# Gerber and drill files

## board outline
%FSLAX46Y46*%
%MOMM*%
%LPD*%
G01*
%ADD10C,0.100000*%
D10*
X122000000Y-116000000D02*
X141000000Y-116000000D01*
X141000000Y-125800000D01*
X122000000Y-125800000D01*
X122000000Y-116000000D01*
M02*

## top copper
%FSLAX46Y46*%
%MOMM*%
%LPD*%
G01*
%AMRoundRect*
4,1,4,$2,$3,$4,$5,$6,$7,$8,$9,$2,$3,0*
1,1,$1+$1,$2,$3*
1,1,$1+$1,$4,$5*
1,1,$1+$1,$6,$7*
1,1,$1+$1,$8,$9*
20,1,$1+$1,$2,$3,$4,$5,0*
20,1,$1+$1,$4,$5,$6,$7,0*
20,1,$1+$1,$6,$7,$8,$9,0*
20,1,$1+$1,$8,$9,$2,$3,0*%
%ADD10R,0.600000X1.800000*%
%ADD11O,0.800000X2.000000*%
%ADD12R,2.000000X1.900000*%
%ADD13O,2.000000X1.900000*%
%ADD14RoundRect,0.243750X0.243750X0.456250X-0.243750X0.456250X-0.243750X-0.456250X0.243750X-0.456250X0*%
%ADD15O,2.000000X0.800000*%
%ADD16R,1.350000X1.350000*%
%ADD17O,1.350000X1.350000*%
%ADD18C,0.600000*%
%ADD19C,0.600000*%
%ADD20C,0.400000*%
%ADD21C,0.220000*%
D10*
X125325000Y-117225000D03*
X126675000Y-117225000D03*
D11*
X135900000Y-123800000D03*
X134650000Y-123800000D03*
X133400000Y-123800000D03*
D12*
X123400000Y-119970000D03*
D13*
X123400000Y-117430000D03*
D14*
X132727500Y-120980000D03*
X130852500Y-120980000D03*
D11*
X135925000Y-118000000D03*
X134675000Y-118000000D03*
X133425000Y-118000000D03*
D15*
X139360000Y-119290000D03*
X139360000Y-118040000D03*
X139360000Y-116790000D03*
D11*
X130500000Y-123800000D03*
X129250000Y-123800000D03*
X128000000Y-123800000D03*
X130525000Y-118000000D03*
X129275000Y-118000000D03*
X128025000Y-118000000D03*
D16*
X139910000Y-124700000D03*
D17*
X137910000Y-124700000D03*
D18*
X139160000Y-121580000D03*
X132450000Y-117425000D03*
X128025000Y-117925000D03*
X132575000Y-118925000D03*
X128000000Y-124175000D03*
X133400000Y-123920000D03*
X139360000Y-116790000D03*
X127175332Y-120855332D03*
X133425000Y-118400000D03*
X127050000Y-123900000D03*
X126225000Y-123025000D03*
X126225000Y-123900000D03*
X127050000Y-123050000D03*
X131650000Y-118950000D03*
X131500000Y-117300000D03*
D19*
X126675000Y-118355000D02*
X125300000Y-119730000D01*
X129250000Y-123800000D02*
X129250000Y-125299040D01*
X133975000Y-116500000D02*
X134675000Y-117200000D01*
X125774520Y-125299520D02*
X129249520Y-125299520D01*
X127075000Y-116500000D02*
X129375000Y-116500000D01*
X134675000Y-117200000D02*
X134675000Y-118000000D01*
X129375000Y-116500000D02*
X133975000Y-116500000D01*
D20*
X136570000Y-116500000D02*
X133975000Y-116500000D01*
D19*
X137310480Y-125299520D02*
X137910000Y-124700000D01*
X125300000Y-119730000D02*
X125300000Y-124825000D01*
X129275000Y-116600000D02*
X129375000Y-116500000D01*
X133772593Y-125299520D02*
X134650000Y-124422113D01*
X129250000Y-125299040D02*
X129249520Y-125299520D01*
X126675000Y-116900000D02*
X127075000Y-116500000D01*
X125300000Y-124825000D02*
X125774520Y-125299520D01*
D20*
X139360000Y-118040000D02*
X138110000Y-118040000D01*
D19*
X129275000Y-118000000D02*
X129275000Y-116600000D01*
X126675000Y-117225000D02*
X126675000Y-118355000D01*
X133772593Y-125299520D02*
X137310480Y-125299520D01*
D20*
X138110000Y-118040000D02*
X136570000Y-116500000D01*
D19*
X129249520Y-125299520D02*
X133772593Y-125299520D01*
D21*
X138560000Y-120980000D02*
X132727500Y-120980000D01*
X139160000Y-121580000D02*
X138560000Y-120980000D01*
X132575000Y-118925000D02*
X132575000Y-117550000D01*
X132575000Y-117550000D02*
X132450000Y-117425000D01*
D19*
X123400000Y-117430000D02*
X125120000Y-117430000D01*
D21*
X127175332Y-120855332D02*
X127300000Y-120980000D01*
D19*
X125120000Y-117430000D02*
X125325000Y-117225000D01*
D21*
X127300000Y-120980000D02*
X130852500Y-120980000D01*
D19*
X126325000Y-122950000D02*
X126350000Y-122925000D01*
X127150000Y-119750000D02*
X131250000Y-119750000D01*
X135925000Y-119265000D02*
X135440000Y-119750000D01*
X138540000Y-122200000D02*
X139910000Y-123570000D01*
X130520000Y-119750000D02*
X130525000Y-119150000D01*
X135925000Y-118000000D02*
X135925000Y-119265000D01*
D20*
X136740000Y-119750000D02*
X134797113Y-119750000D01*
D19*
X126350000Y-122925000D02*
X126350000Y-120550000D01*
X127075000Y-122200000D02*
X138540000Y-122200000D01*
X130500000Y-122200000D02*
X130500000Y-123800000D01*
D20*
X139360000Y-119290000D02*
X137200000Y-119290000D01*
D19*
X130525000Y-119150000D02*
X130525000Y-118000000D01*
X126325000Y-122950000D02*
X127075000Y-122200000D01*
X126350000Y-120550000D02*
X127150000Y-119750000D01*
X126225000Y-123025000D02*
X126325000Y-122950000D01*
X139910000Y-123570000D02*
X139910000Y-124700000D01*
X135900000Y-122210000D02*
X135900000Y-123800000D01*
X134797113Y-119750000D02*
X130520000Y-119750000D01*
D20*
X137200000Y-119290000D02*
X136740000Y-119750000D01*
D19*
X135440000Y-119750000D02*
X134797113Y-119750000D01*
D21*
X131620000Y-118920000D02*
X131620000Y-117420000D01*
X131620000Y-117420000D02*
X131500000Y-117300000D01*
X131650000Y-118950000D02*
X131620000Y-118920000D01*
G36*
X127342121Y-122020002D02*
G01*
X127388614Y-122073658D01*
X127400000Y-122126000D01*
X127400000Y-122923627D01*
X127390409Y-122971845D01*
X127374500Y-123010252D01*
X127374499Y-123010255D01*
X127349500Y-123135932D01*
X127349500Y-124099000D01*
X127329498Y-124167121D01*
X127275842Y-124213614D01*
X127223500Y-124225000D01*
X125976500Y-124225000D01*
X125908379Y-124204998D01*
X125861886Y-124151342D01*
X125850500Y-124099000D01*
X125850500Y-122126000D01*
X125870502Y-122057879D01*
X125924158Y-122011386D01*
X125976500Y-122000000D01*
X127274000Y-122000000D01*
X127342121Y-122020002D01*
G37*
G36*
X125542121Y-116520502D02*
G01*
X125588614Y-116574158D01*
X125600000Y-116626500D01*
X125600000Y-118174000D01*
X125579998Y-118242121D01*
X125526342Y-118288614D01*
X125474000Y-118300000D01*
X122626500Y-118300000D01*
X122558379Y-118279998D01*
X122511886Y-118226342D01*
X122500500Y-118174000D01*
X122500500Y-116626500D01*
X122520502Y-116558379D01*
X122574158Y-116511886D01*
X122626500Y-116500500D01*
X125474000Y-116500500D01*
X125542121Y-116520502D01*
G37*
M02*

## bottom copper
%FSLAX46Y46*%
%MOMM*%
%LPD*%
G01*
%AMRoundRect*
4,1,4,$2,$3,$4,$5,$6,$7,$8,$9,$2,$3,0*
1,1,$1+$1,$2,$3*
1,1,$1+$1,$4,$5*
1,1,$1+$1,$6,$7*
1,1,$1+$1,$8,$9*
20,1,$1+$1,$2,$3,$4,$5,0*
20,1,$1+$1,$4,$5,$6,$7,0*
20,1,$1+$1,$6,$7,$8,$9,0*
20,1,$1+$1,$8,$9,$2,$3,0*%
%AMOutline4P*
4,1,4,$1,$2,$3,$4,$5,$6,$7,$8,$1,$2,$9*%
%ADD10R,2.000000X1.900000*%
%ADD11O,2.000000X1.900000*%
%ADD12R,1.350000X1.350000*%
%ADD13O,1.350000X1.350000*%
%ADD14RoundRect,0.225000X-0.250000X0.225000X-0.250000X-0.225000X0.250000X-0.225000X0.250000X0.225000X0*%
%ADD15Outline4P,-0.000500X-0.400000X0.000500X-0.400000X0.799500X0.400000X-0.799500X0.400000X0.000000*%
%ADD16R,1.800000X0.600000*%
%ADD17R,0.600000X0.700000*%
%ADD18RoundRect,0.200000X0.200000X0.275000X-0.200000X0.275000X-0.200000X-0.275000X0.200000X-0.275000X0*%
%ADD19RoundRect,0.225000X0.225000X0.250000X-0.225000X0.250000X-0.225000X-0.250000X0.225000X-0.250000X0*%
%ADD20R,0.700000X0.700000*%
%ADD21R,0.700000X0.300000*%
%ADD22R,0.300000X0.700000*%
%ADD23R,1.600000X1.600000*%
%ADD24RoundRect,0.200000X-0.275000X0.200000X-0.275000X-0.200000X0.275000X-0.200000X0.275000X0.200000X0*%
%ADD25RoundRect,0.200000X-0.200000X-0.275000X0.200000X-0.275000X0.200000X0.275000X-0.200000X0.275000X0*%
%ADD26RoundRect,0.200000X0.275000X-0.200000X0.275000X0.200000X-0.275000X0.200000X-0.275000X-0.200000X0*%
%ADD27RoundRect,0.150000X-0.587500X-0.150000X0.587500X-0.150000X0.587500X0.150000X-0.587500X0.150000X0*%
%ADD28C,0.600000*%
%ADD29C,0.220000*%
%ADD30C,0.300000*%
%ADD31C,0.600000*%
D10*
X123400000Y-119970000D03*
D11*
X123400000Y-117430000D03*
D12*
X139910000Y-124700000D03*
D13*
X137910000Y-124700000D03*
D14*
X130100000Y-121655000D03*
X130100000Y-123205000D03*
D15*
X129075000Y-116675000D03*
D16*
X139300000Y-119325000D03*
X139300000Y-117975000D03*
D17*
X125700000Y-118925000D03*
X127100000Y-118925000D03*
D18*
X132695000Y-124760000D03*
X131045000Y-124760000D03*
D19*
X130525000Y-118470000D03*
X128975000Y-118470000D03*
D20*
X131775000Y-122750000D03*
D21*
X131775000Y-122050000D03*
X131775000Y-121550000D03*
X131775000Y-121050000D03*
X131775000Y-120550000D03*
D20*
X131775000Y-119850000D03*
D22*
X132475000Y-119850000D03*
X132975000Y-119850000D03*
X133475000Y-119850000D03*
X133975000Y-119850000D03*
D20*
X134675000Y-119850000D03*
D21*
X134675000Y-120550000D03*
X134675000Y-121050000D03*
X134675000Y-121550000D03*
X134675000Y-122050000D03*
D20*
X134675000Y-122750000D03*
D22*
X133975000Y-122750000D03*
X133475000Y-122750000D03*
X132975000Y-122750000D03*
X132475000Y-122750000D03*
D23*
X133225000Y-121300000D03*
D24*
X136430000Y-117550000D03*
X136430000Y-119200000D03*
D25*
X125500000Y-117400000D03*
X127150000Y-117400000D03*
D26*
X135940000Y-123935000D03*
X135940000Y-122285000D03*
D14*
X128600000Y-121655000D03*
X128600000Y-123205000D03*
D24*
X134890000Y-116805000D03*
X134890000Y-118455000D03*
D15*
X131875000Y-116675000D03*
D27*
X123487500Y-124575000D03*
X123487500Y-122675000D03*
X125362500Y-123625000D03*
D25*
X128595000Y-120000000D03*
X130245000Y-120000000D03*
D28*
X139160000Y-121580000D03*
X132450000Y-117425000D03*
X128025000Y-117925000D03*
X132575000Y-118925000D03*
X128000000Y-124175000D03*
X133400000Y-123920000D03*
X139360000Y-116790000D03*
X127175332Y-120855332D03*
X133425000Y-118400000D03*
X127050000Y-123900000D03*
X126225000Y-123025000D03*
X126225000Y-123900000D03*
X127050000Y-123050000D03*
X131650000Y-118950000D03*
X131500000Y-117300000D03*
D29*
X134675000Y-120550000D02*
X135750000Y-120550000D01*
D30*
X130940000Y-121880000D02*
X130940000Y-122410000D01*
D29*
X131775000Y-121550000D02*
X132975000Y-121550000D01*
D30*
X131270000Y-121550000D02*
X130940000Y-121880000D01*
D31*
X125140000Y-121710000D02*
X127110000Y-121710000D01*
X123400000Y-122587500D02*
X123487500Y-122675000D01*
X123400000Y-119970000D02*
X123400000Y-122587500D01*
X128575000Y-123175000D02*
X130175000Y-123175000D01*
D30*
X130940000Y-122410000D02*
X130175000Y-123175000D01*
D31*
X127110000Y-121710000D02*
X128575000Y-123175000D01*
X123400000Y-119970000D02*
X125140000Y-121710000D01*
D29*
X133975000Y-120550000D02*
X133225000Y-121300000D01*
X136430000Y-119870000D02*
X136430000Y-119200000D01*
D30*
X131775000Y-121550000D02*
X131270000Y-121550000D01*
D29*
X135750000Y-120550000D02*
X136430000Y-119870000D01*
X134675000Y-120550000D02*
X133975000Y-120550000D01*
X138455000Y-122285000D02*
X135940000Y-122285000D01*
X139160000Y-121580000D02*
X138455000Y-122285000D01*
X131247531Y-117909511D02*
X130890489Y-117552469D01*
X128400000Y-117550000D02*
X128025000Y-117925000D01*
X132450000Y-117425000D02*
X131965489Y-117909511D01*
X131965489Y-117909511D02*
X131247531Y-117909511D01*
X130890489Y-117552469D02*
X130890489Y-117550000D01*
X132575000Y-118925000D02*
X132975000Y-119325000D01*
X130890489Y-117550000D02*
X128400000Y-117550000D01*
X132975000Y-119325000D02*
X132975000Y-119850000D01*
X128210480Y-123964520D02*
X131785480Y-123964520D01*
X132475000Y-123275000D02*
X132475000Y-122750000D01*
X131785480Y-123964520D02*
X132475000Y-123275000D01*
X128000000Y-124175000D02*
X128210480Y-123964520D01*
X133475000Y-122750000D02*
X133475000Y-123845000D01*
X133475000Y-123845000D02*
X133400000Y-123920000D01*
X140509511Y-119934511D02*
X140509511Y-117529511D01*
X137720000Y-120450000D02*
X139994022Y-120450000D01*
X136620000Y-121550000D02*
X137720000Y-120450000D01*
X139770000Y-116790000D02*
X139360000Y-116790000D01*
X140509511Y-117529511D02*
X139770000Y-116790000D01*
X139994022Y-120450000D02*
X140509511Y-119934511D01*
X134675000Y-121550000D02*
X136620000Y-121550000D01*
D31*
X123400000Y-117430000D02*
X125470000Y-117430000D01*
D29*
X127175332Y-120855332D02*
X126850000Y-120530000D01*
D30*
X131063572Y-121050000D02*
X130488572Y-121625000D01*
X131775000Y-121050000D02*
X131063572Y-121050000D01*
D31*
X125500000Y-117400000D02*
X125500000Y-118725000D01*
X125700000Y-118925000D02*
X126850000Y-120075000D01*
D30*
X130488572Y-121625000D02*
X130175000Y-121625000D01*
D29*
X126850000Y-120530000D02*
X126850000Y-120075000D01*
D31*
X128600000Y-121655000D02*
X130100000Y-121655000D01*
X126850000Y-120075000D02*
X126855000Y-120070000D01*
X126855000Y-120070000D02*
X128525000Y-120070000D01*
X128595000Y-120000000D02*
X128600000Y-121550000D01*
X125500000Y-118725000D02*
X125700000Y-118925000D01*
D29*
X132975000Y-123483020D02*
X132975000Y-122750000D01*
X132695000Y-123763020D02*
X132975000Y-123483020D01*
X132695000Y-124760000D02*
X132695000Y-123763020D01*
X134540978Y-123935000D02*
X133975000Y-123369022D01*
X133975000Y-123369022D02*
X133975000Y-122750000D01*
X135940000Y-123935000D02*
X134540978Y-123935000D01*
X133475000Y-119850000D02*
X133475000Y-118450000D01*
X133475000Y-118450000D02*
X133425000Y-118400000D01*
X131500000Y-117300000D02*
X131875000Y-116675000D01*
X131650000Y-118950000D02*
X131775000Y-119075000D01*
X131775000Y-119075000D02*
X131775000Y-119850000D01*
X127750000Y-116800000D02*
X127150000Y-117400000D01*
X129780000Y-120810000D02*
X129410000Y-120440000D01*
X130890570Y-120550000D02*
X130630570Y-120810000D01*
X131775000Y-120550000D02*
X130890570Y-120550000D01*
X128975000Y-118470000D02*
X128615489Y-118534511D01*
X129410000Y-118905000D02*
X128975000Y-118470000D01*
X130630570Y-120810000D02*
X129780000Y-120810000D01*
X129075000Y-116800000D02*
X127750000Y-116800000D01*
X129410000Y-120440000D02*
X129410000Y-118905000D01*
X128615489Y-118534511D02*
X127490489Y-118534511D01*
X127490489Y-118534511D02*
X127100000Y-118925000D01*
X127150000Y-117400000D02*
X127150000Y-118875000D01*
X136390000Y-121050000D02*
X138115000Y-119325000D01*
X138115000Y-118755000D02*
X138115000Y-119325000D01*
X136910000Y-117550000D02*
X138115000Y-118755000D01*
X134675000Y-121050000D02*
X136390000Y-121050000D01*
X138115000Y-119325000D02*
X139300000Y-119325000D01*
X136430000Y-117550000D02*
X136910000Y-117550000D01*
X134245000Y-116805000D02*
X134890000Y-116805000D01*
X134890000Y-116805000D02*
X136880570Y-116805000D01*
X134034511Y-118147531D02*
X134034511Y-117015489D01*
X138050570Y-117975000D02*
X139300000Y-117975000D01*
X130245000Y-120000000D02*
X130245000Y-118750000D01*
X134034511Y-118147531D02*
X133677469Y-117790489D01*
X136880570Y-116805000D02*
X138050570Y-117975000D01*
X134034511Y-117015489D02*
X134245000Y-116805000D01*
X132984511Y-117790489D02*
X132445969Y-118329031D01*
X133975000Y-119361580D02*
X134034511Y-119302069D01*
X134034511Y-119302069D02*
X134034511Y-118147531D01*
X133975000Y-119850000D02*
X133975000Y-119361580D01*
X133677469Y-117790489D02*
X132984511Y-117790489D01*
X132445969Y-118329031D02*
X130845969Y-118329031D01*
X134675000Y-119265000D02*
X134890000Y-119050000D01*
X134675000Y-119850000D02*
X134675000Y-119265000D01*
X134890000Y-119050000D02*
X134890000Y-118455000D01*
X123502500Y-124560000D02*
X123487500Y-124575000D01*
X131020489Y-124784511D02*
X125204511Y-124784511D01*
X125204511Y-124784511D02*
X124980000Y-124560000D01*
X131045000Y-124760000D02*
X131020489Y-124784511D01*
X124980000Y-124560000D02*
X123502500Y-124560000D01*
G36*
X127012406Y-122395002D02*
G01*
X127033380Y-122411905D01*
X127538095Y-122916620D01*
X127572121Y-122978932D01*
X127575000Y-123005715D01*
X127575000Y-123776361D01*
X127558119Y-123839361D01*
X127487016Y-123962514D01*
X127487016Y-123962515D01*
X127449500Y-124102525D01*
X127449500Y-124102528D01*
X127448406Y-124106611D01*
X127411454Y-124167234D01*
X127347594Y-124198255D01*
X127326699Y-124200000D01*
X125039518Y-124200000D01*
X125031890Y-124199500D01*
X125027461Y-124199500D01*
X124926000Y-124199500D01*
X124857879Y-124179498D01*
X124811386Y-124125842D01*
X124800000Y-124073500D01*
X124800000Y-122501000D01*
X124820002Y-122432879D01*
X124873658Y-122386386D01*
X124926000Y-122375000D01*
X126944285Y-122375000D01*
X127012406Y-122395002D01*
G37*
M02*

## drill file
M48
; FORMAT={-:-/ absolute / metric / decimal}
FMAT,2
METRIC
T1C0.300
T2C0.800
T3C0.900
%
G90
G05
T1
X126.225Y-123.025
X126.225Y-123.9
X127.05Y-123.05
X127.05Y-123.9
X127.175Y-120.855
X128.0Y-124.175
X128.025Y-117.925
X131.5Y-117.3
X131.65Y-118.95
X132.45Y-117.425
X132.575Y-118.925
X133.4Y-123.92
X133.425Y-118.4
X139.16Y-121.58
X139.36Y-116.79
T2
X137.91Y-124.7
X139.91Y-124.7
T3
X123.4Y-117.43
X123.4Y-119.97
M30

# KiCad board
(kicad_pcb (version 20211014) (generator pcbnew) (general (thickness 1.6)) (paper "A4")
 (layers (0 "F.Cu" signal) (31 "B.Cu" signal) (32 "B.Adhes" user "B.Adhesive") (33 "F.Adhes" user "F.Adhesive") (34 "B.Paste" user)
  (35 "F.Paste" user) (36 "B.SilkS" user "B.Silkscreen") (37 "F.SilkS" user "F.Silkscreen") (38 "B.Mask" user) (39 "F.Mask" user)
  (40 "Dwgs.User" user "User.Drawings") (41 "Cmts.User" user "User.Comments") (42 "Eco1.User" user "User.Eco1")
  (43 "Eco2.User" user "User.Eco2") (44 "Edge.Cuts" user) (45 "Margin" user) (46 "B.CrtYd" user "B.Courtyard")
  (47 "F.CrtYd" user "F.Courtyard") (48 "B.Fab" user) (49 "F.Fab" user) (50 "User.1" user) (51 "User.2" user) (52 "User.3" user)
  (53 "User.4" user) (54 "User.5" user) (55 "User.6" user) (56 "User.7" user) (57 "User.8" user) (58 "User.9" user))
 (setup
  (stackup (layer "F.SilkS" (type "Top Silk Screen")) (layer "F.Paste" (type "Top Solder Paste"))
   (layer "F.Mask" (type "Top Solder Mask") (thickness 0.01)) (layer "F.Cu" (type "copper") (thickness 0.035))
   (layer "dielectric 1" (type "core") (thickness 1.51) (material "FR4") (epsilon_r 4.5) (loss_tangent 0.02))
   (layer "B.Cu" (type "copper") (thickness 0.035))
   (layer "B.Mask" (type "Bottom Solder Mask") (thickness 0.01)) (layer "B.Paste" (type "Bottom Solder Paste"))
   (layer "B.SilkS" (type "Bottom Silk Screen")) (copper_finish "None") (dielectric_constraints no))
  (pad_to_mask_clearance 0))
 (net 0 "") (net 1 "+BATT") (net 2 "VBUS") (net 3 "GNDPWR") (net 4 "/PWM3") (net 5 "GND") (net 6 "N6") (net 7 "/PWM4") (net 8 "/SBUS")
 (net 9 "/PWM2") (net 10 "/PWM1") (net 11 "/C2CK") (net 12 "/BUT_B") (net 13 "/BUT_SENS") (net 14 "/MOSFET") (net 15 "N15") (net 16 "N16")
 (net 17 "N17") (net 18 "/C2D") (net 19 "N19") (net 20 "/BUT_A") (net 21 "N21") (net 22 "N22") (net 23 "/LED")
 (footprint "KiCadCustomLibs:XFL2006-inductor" (layer "F.Cu") (at 126 117.225)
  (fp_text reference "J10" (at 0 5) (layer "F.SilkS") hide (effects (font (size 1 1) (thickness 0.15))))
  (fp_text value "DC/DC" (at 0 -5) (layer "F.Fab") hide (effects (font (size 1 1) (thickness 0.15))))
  (pad "1" smd rect locked (at -0.675 0) (size 0.6 1.8) (layers "F.Cu" "F.Paste" "F.Mask") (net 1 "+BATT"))
  (pad "2" smd rect locked (at 0.675 0) (size 0.6 1.8) (layers "F.Cu" "F.Paste" "F.Mask") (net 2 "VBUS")))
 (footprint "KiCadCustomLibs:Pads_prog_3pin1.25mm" (layer "F.Cu") (at 134.675 123.8 180)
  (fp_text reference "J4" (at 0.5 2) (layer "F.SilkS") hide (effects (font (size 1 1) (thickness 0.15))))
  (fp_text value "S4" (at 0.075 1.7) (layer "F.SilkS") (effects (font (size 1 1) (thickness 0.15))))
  (pad "1" smd oval locked (at -1.225 0 180) (size 0.8 2) (layers "F.Cu" "F.Paste" "F.Mask") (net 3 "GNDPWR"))
  (pad "2" smd oval locked (at 0.025 0 180) (size 0.8 2) (layers "F.Cu" "F.Paste" "F.Mask") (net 2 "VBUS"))
  (pad "3" smd oval locked (at 1.275 0 180) (size 0.8 2) (layers "F.Cu" "F.Paste" "F.Mask") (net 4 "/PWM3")))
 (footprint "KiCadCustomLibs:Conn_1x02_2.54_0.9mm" (layer "F.Cu") (at 123.4 119.97 180)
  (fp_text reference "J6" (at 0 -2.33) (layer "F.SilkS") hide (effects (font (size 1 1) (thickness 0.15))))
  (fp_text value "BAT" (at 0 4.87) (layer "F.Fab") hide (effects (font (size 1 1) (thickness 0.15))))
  (pad "1" thru_hole rect locked (at 0 0 180) (size 2 1.9) (drill 0.9) (layers *.Cu *.Mask) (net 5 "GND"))
  (pad "2" thru_hole oval locked (at 0 2.54 180) (size 2 1.9) (drill 0.9) (layers *.Cu *.Mask) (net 1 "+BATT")))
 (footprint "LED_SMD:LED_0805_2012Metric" (layer "F.Cu") (at 131.79 120.98 180)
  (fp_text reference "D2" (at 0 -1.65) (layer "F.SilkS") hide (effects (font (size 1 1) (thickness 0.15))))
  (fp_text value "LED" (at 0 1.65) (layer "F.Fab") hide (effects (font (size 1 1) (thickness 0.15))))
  (pad "1" smd roundrect (at -0.9375 0 180) (size 0.975 1.4) (layers "F.Cu" "F.Paste" "F.Mask") (roundrect_rratio 0.25) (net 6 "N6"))
  (pad "2" smd roundrect (at 0.9375 0 180) (size 0.975 1.4) (layers "F.Cu" "F.Paste" "F.Mask") (roundrect_rratio 0.25) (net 1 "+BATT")))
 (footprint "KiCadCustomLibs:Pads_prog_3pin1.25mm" (layer "F.Cu") (at 134.7 118 180)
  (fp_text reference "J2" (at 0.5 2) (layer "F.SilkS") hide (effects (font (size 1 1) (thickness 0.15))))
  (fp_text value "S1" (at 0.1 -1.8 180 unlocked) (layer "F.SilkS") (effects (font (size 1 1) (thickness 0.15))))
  (pad "1" smd oval locked (at -1.225 0 180) (size 0.8 2) (layers "F.Cu" "F.Paste" "F.Mask") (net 3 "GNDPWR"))
  (pad "2" smd oval locked (at 0.025 0 180) (size 0.8 2) (layers "F.Cu" "F.Paste" "F.Mask") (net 2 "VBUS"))
  (pad "3" smd oval locked (at 1.275 0 180) (size 0.8 2) (layers "F.Cu" "F.Paste" "F.Mask") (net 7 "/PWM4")))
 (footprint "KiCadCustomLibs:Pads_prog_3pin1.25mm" (layer "F.Cu") (at 139.36 118.065 90)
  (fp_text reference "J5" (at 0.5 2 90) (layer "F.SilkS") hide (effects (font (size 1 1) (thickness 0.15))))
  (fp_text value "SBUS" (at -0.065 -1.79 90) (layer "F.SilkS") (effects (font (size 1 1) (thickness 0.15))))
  (pad "1" smd oval locked (at -1.225 0 90) (size 0.8 2) (layers "F.Cu" "F.Paste" "F.Mask") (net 3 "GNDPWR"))
  (pad "2" smd oval locked (at 0.025 0 90) (size 0.8 2) (layers "F.Cu" "F.Paste" "F.Mask") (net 2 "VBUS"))
  (pad "3" smd oval locked (at 1.275 0 90) (size 0.8 2) (layers "F.Cu" "F.Paste" "F.Mask") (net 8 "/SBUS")))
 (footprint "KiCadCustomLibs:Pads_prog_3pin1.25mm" (layer "F.Cu") (at 129.275 123.8 180)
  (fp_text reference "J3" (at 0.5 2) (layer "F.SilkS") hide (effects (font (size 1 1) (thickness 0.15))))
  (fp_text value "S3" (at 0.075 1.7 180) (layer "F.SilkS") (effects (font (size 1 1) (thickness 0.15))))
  (pad "1" smd oval locked (at -1.225 0 180) (size 0.8 2) (layers "F.Cu" "F.Paste" "F.Mask") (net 3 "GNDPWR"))
  (pad "2" smd oval locked (at 0.025 0 180) (size 0.8 2) (layers "F.Cu" "F.Paste" "F.Mask") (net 2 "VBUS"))
  (pad "3" smd oval locked (at 1.275 0 180) (size 0.8 2) (layers "F.Cu" "F.Paste" "F.Mask") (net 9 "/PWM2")))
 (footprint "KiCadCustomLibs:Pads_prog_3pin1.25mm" (layer "F.Cu") (at 129.3 118 180)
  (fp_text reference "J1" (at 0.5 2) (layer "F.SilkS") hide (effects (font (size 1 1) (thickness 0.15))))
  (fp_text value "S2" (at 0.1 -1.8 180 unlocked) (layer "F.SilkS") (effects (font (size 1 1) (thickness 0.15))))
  (pad "1" smd oval locked (at -1.225 0 180) (size 0.8 2) (layers "F.Cu" "F.Paste" "F.Mask") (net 3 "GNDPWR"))
  (pad "2" smd oval locked (at 0.025 0 180) (size 0.8 2) (layers "F.Cu" "F.Paste" "F.Mask") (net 2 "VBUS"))
  (pad "3" smd oval locked (at 1.275 0 180) (size 0.8 2) (layers "F.Cu" "F.Paste" "F.Mask") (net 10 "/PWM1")))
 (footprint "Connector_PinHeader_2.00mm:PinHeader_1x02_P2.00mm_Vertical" (layer "B.Cu") (at 139.91 124.7 90)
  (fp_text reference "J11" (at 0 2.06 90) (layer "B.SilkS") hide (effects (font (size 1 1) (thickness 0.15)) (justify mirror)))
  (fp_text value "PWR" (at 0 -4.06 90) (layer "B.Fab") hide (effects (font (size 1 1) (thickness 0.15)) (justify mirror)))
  (pad "1" thru_hole rect (at 0 0 90) (size 1.35 1.35) (drill 0.8) (layers *.Cu *.Mask) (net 3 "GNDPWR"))
  (pad "2" thru_hole oval (at 0 -2 90) (size 1.35 1.35) (drill 0.8) (layers *.Cu *.Mask) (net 2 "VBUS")))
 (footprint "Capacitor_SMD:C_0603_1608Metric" (layer "B.Cu") (at 130.1 122.43 -90)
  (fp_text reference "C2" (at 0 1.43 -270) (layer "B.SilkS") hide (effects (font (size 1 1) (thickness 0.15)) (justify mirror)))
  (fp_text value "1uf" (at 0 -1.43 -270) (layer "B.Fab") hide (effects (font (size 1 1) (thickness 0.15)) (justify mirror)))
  (pad "1" smd roundrect (at -0.775 0 270) (size 0.9 0.95) (layers "B.Cu" "B.Paste" "B.Mask") (roundrect_rratio 0.25) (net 1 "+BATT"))
  (pad "2" smd roundrect (at 0.775 0 270) (size 0.9 0.95) (layers "B.Cu" "B.Paste" "B.Mask") (roundrect_rratio 0.25) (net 5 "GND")))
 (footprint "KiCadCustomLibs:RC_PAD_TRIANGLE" (layer "B.Cu") (at 129.075 116.675)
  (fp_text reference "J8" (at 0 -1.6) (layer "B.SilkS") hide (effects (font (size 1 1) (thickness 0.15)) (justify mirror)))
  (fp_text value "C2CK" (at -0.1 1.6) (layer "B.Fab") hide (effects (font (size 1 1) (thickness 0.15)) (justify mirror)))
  (pad "1" smd trapezoid locked (at 0 0) (size 0.8 0.8) (rect_delta 0 -0.799) (layers "B.Cu" "B.Paste" "B.Mask") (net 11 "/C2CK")))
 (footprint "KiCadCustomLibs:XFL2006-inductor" (layer "B.Cu") (at 139.3 118.65 90)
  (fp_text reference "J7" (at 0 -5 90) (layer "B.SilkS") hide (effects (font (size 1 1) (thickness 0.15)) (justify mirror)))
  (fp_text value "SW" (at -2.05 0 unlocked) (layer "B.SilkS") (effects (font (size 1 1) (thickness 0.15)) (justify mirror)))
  (pad "1" smd rect locked (at -0.675 0 90) (size 0.6 1.8) (layers "B.Cu" "B.Paste" "B.Mask") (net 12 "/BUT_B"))
  (pad "2" smd rect locked (at 0.675 0 90) (size 0.6 1.8) (layers "B.Cu" "B.Paste" "B.Mask") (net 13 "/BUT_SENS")))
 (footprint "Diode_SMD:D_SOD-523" (layer "B.Cu") (at 126.4 118.925)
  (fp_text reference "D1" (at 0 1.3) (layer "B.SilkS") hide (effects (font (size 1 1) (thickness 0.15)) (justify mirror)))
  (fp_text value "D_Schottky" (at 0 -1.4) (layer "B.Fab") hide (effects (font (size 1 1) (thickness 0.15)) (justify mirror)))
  (pad "1" smd rect (at -0.7 0 180) (size 0.6 0.7) (layers "B.Cu" "B.Paste" "B.Mask") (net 1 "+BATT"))
  (pad "2" smd rect (at 0.7 0 180) (size 0.6 0.7) (layers "B.Cu" "B.Paste" "B.Mask") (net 11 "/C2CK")))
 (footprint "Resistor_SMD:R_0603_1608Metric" (layer "B.Cu") (at 131.87 124.76 180)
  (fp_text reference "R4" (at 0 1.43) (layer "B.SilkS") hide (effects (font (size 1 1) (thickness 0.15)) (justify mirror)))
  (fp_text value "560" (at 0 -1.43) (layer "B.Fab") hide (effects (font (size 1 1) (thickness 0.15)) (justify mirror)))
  (pad "1" smd roundrect (at -0.825 0 180) (size 0.8 0.95) (layers "B.Cu" "B.Paste" "B.Mask") (roundrect_rratio 0.25) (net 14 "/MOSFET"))
  (pad "2" smd roundrect (at 0.825 0 180) (size 0.8 0.95) (layers "B.Cu" "B.Paste" "B.Mask") (roundrect_rratio 0.25) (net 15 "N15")))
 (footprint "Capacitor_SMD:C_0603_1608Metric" (layer "B.Cu") (at 129.75 118.47 180)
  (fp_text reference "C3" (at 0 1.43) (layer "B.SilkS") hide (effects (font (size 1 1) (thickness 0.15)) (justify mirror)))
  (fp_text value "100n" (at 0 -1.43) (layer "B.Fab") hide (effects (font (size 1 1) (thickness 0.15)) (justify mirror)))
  (pad "1" smd roundrect (at -0.775 0 180) (size 0.9 0.95) (layers "B.Cu" "B.Paste" "B.Mask") (roundrect_rratio 0.25) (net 13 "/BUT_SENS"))
  (pad "2" smd roundrect (at 0.775 0 180) (size 0.9 0.95) (layers "B.Cu" "B.Paste" "B.Mask") (roundrect_rratio 0.25) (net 11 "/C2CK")))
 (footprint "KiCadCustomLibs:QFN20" (layer "B.Cu") (at 133.225 121.3 90)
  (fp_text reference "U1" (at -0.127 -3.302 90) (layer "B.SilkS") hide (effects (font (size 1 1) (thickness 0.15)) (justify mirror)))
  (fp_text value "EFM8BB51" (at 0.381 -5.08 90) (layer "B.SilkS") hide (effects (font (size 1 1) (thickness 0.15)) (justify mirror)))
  (pad "1" smd rect locked (at -1.45 -1.45 90) (size 0.7 0.7) (layers "B.Cu" "B.Paste" "B.Mask") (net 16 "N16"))
  (pad "2" smd rect locked (at -0.75 -1.45 90) (size 0.3 0.7) (layers "B.Cu" "B.Paste" "B.Mask") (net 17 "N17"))
  (pad "3" smd rect locked (at -0.25 -1.45 90) (size 0.3 0.7) (layers "B.Cu" "B.Paste" "B.Mask") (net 5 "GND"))
  (pad "4" smd rect locked (at 0.25 -1.45 90) (size 0.3 0.7) (layers "B.Cu" "B.Paste" "B.Mask") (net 1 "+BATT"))
  (pad "5" smd rect locked (at 0.75 -1.45 90) (size 0.3 0.7) (layers "B.Cu" "B.Paste" "B.Mask") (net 11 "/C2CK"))
  (pad "6" smd rect locked (at 1.45 -1.45 90) (size 0.7 0.7) (layers "B.Cu" "B.Paste" "B.Mask") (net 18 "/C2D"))
  (pad "7" smd rect locked (at 1.45 -0.75) (size 0.3 0.7) (layers "B.Cu" "B.Paste" "B.Mask") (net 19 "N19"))
  (pad "8" smd rect locked (at 1.45 -0.25) (size 0.3 0.7) (layers "B.Cu" "B.Paste" "B.Mask") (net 10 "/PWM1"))
  (pad "9" smd rect locked (at 1.45 0.25) (size 0.3 0.7) (layers "B.Cu" "B.Paste" "B.Mask") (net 7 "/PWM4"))
  (pad "10" smd rect locked (at 1.45 0.75) (size 0.3 0.7) (layers "B.Cu" "B.Paste" "B.Mask") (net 13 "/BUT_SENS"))
  (pad "11" smd rect locked (at 1.45 1.45 90) (size 0.7 0.7) (layers "B.Cu" "B.Paste" "B.Mask") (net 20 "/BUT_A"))
  (pad "12" smd rect locked (at 0.75 1.45 90) (size 0.3 0.7) (layers "B.Cu" "B.Paste" "B.Mask") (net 5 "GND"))
  (pad "13" smd rect locked (at 0.25 1.45 90) (size 0.3 0.7) (layers "B.Cu" "B.Paste" "B.Mask") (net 12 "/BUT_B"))
  (pad "14" smd rect locked (at -0.25 1.45 90) (size 0.3 0.7) (layers "B.Cu" "B.Paste" "B.Mask") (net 8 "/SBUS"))
  (pad "15" smd rect locked (at -0.75 1.45 90) (size 0.3 0.7) (layers "B.Cu" "B.Paste" "B.Mask") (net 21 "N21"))
  (pad "16" smd rect locked (at -1.45 1.45 90) (size 0.7 0.7) (layers "B.Cu" "B.Paste" "B.Mask") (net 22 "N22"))
  (pad "17" smd rect locked (at -1.45 0.75) (size 0.3 0.7) (layers "B.Cu" "B.Paste" "B.Mask") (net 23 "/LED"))
  (pad "18" smd rect locked (at -1.45 0.25) (size 0.3 0.7) (layers "B.Cu" "B.Paste" "B.Mask") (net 4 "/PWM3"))
  (pad "19" smd rect locked (at -1.45 -0.25) (size 0.3 0.7) (layers "B.Cu" "B.Paste" "B.Mask") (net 14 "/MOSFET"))
  (pad "20" smd rect locked (at -1.45 -0.75) (size 0.3 0.7) (layers "B.Cu" "B.Paste" "B.Mask") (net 9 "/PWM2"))
  (pad "21" smd rect locked (at 0 0 90) (size 1.6 1.6) (layers "B.Cu" "B.Paste" "B.Mask") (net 5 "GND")))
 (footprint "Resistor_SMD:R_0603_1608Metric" (layer "B.Cu") (at 136.43 118.375 -90)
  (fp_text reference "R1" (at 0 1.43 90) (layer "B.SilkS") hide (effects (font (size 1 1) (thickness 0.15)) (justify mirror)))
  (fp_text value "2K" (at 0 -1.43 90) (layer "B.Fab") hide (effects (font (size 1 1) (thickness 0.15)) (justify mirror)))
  (pad "1" smd roundrect (at -0.825 0 270) (size 0.8 0.95) (layers "B.Cu" "B.Paste" "B.Mask") (roundrect_rratio 0.25) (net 12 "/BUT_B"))
  (pad "2" smd roundrect (at 0.825 0 270) (size 0.8 0.95) (layers "B.Cu" "B.Paste" "B.Mask") (roundrect_rratio 0.25) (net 5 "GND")))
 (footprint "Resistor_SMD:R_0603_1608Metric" (layer "B.Cu") (at 126.325 117.4)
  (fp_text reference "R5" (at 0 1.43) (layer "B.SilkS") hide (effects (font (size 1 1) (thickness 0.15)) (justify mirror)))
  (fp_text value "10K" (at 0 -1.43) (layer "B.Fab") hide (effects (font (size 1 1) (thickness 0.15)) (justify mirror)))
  (pad "1" smd roundrect (at -0.825 0) (size 0.8 0.95) (layers "B.Cu" "B.Paste" "B.Mask") (roundrect_rratio 0.25) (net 1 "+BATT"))
  (pad "2" smd roundrect (at 0.825 0) (size 0.8 0.95) (layers "B.Cu" "B.Paste" "B.Mask") (roundrect_rratio 0.25) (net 11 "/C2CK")))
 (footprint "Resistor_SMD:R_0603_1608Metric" (layer "B.Cu") (at 135.94 123.11 90)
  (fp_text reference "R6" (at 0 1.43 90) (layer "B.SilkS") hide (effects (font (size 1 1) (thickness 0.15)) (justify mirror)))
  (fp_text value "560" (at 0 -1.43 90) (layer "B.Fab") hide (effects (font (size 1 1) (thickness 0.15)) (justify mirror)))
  (pad "1" smd roundrect (at -0.825 0 90) (size 0.8 0.95) (layers "B.Cu" "B.Paste" "B.Mask") (roundrect_rratio 0.25) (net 23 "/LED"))
  (pad "2" smd roundrect (at 0.825 0 90) (size 0.8 0.95) (layers "B.Cu" "B.Paste" "B.Mask") (roundrect_rratio 0.25) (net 6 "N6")))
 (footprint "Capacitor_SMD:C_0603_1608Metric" (layer "B.Cu") (at 128.6 122.43 -90)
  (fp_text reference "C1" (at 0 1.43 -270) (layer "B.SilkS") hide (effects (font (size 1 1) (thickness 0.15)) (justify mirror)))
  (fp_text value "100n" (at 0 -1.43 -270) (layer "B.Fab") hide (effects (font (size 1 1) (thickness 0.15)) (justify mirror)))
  (pad "1" smd roundrect (at -0.775 0 270) (size 0.9 0.95) (layers "B.Cu" "B.Paste" "B.Mask") (roundrect_rratio 0.25) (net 1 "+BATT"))
  (pad "2" smd roundrect (at 0.775 0 270) (size 0.9 0.95) (layers "B.Cu" "B.Paste" "B.Mask") (roundrect_rratio 0.25) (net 5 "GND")))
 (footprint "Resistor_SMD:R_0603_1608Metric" (layer "B.Cu") (at 134.89 117.63 -90)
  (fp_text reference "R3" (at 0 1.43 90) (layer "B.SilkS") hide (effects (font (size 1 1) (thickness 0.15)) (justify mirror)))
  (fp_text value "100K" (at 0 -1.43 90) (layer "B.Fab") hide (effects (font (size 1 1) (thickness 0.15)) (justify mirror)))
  (pad "1" smd roundrect (at -0.825 0 270) (size 0.8 0.95) (layers "B.Cu" "B.Paste" "B.Mask") (roundrect_rratio 0.25) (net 13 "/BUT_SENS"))
  (pad "2" smd roundrect (at 0.825 0 270) (size 0.8 0.95) (layers "B.Cu" "B.Paste" "B.Mask") (roundrect_rratio 0.25) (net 20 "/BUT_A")))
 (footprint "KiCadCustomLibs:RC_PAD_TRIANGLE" (layer "B.Cu") (at 131.875 116.675)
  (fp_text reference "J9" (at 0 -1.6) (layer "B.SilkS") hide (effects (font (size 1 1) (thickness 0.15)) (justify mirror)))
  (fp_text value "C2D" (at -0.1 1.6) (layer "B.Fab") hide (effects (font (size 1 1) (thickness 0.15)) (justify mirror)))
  (pad "1" smd trapezoid locked (at 0 0) (size 0.8 0.8) (rect_delta 0 -0.799) (layers "B.Cu" "B.Paste" "B.Mask") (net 18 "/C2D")))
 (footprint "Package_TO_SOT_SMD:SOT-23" (layer "B.Cu") (at 124.425 123.625)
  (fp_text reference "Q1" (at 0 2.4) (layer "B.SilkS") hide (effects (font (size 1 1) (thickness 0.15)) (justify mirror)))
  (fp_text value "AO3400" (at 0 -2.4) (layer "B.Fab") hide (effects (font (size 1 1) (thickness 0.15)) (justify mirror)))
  (pad "1" smd roundrect (at -0.9375 0.95) (size 1.475 0.6) (layers "B.Cu" "B.Paste" "B.Mask") (roundrect_rratio 0.25) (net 15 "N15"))
  (pad "2" smd roundrect (at -0.9375 -0.95) (size 1.475 0.6) (layers "B.Cu" "B.Paste" "B.Mask") (roundrect_rratio 0.25) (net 5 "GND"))
  (pad "3" smd roundrect (at 0.9375 0) (size 1.475 0.6) (layers "B.Cu" "B.Paste" "B.Mask") (roundrect_rratio 0.25) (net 3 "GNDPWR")))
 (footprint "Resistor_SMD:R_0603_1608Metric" (layer "B.Cu") (at 129.42 120)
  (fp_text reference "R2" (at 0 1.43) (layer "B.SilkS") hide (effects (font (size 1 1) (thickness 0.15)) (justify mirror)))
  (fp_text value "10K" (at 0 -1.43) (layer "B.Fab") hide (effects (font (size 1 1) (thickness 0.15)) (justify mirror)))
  (pad "1" smd roundrect (at -0.825 0) (size 0.8 0.95) (layers "B.Cu" "B.Paste" "B.Mask") (roundrect_rratio 0.25) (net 1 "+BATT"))
  (pad "2" smd roundrect (at 0.825 0) (size 0.8 0.95) (layers "B.Cu" "B.Paste" "B.Mask") (roundrect_rratio 0.25) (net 13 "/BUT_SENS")))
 (gr_rect (start 122 116) (end 141 125.8) (layer "Edge.Cuts") (width 0.1) (fill none))
 (segment (start 126.675 118.355) (end 125.3 119.73) (width 0.6) (layer "F.Cu") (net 2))
 (segment (start 129.25 123.8) (end 129.25 125.29904) (width 0.6) (layer "F.Cu") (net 2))
 (segment (start 133.975 116.5) (end 134.675 117.2) (width 0.6) (layer "F.Cu") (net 2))
 (segment (start 125.77452 125.29952) (end 129.24952 125.29952) (width 0.6) (layer "F.Cu") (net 2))
 (segment (start 127.075 116.5) (end 129.375 116.5) (width 0.6) (layer "F.Cu") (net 2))
 (segment (start 134.675 117.2) (end 134.675 118) (width 0.6) (layer "F.Cu") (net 2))
 (segment (start 129.375 116.5) (end 133.975 116.5) (width 0.6) (layer "F.Cu") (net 2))
 (segment (start 136.57 116.5) (end 133.975 116.5) (width 0.4) (layer "F.Cu") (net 2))
 (segment (start 137.31048 125.29952) (end 137.91 124.7) (width 0.6) (layer "F.Cu") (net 2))
 (segment (start 125.3 119.73) (end 125.3 124.825) (width 0.6) (layer "F.Cu") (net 2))
 (segment (start 129.275 116.6) (end 129.375 116.5) (width 0.6) (layer "F.Cu") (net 2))
 (segment (start 133.772593 125.29952) (end 134.65 124.422113) (width 0.6) (layer "F.Cu") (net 2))
 (segment (start 129.25 125.29904) (end 129.24952 125.29952) (width 0.6) (layer "F.Cu") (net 2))
 (segment (start 126.675 116.9) (end 127.075 116.5) (width 0.6) (layer "F.Cu") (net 2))
 (segment (start 125.3 124.825) (end 125.77452 125.29952) (width 0.6) (layer "F.Cu") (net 2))
 (segment (start 139.36 118.04) (end 138.11 118.04) (width 0.4) (layer "F.Cu") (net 2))
 (segment (start 129.275 118) (end 129.275 116.6) (width 0.6) (layer "F.Cu") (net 2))
 (segment (start 126.675 117.225) (end 126.675 118.355) (width 0.6) (layer "F.Cu") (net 2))
 (segment (start 133.772593 125.29952) (end 137.31048 125.29952) (width 0.6) (layer "F.Cu") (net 2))
 (segment (start 138.11 118.04) (end 136.57 116.5) (width 0.4) (layer "F.Cu") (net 2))
 (segment (start 129.24952 125.29952) (end 133.772593 125.29952) (width 0.6) (layer "F.Cu") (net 2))
 (segment (start 134.675 120.55) (end 135.75 120.55) (width 0.22) (layer "B.Cu") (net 5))
 (segment (start 130.94 121.88) (end 130.94 122.41) (width 0.3) (layer "B.Cu") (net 5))
 (segment (start 131.775 121.55) (end 132.975 121.55) (width 0.22) (layer "B.Cu") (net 5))
 (segment (start 131.27 121.55) (end 130.94 121.88) (width 0.3) (layer "B.Cu") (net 5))
 (segment (start 125.14 121.71) (end 127.11 121.71) (width 0.6) (layer "B.Cu") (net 5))
 (segment (start 123.4 122.5875) (end 123.4875 122.675) (width 0.6) (layer "B.Cu") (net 5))
 (segment (start 123.4 119.97) (end 123.4 122.5875) (width 0.6) (layer "B.Cu") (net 5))
 (segment (start 128.575 123.175) (end 130.175 123.175) (width 0.6) (layer "B.Cu") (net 5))
 (segment (start 130.94 122.41) (end 130.175 123.175) (width 0.3) (layer "B.Cu") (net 5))
 (segment (start 127.11 121.71) (end 128.575 123.175) (width 0.6) (layer "B.Cu") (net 5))
 (segment (start 123.4 119.97) (end 125.14 121.71) (width 0.6) (layer "B.Cu") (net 5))
 (segment (start 133.975 120.55) (end 133.225 121.3) (width 0.22) (layer "B.Cu") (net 5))
 (segment (start 136.43 119.87) (end 136.43 119.2) (width 0.22) (layer "B.Cu") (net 5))
 (segment (start 131.775 121.55) (end 131.27 121.55) (width 0.3) (layer "B.Cu") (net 5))
 (segment (start 135.75 120.55) (end 136.43 119.87) (width 0.22) (layer "B.Cu") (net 5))
 (segment (start 134.675 120.55) (end 133.975 120.55) (width 0.22) (layer "B.Cu") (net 5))
 (segment (start 138.56 120.98) (end 132.7275 120.98) (width 0.22) (layer "F.Cu") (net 6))
 (segment (start 139.16 121.58) (end 138.56 120.98) (width 0.22) (layer "F.Cu") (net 6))
 (via (at 139.16 121.58) (size 0.6) (drill 0.3) (layers "F.Cu" "B.Cu") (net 6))
 (segment (start 138.455 122.285) (end 135.94 122.285) (width 0.22) (layer "B.Cu") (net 6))
 (segment (start 139.16 121.58) (end 138.455 122.285) (width 0.22) (layer "B.Cu") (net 6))
 (segment (start 132.575 118.925) (end 132.575 117.55) (width 0.22) (layer "F.Cu") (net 10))
 (segment (start 132.575 117.55) (end 132.45 117.425) (width 0.22) (layer "F.Cu") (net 10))
 (via (at 132.45 117.425) (size 0.6) (drill 0.3) (layers "F.Cu" "B.Cu") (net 10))
 (via (at 128.025 117.925) (size 0.6) (drill 0.3) (layers "F.Cu" "B.Cu") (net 10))
 (via (at 132.575 118.925) (size 0.6) (drill 0.3) (layers "F.Cu" "B.Cu") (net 10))
 (segment (start 131.247531 117.909511) (end 130.890489 117.552469) (width 0.22) (layer "B.Cu") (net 10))
 (segment (start 128.4 117.55) (end 128.025 117.925) (width 0.22) (layer "B.Cu") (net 10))
 (segment (start 132.45 117.425) (end 131.965489 117.909511) (width 0.22) (layer "B.Cu") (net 10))
 (segment (start 131.965489 117.909511) (end 131.247531 117.909511) (width 0.22) (layer "B.Cu") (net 10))
 (segment (start 130.890489 117.552469) (end 130.890489 117.55) (width 0.22) (layer "B.Cu") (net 10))
 (segment (start 132.575 118.925) (end 132.975 119.325) (width 0.22) (layer "B.Cu") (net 10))
 (segment (start 130.890489 117.55) (end 128.4 117.55) (width 0.22) (layer "B.Cu") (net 10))
 (segment (start 132.975 119.325) (end 132.975 119.85) (width 0.22) (layer "B.Cu") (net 10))
 (via (at 128 124.175) (size 0.6) (drill 0.3) (layers "F.Cu" "B.Cu") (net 9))
 (segment (start 128.21048 123.96452) (end 131.78548 123.96452) (width 0.22) (layer "B.Cu") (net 9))
 (segment (start 132.475 123.275) (end 132.475 122.75) (width 0.22) (layer "B.Cu") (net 9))
 (segment (start 131.78548 123.96452) (end 132.475 123.275) (width 0.22) (layer "B.Cu") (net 9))
 (segment (start 128 124.175) (end 128.21048 123.96452) (width 0.22) (layer "B.Cu") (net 9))
 (via (at 133.4 123.92) (size 0.6) (drill 0.3) (layers "F.Cu" "B.Cu") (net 4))
 (segment (start 133.475 122.75) (end 133.475 123.845) (width 0.22) (layer "B.Cu") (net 4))
 (segment (start 133.475 123.845) (end 133.4 123.92) (width 0.22) (layer "B.Cu") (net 4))
 (via (at 139.36 116.79) (size 0.6) (drill 0.3) (layers "F.Cu" "B.Cu") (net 8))
 (segment (start 140.509511 119.934511) (end 140.509511 117.529511) (width 0.22) (layer "B.Cu") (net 8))
 (segment (start 137.72 120.45) (end 139.994022 120.45) (width 0.22) (layer "B.Cu") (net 8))
 (segment (start 136.62 121.55) (end 137.72 120.45) (width 0.22) (layer "B.Cu") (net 8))
 (segment (start 139.77 116.79) (end 139.36 116.79) (width 0.22) (layer "B.Cu") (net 8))
 (segment (start 140.509511 117.529511) (end 139.77 116.79) (width 0.22) (layer "B.Cu") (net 8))
 (segment (start 139.994022 120.45) (end 140.509511 119.934511) (width 0.22) (layer "B.Cu") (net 8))
 (segment (start 134.675 121.55) (end 136.62 121.55) (width 0.22) (layer "B.Cu") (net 8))
 (segment (start 123.4 117.43) (end 125.12 117.43) (width 0.6) (layer "F.Cu") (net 1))
 (segment (start 127.175332 120.855332) (end 127.3 120.98) (width 0.22) (layer "F.Cu") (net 1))
 (segment (start 125.12 117.43) (end 125.325 117.225) (width 0.6) (layer "F.Cu") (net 1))
 (segment (start 127.3 120.98) (end 130.8525 120.98) (width 0.22) (layer "F.Cu") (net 1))
 (via (at 127.175332 120.855332) (size 0.6) (drill 0.3) (layers "F.Cu" "B.Cu") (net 1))
 (segment (start 123.4 117.43) (end 125.47 117.43) (width 0.6) (layer "B.Cu") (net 1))
 (segment (start 127.175332 120.855332) (end 126.85 120.53) (width 0.22) (layer "B.Cu") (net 1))
 (segment (start 131.063572 121.05) (end 130.488572 121.625) (width 0.3) (layer "B.Cu") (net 1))
 (segment (start 131.775 121.05) (end 131.063572 121.05) (width 0.3) (layer "B.Cu") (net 1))
 (segment (start 125.5 117.4) (end 125.5 118.725) (width 0.6) (layer "B.Cu") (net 1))
 (segment (start 125.7 118.925) (end 126.85 120.075) (width 0.6) (layer "B.Cu") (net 1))
 (segment (start 130.488572 121.625) (end 130.175 121.625) (width 0.3) (layer "B.Cu") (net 1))
 (segment (start 126.85 120.53) (end 126.85 120.075) (width 0.22) (layer "B.Cu") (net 1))
 (segment (start 128.6 121.655) (end 130.1 121.655) (width 0.6) (layer "B.Cu") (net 1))
 (segment (start 126.85 120.075) (end 126.855 120.07) (width 0.6) (layer "B.Cu") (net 1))
 (segment (start 126.855 120.07) (end 128.525 120.07) (width 0.6) (layer "B.Cu") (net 1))
 (segment (start 128.595 120) (end 128.6 121.55) (width 0.6) (layer "B.Cu") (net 1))
 (segment (start 125.5 118.725) (end 125.7 118.925) (width 0.6) (layer "B.Cu") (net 1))
 (segment (start 132.975 123.48302) (end 132.975 122.75) (width 0.22) (layer "B.Cu") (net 14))
 (segment (start 132.695 123.76302) (end 132.975 123.48302) (width 0.22) (layer "B.Cu") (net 14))
 (segment (start 132.695 124.76) (end 132.695 123.76302) (width 0.22) (layer "B.Cu") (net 14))
 (segment (start 134.540978 123.935) (end 133.975 123.369022) (width 0.22) (layer "B.Cu") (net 23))
 (segment (start 133.975 123.369022) (end 133.975 122.75) (width 0.22) (layer "B.Cu") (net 23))
 (segment (start 135.94 123.935) (end 134.540978 123.935) (width 0.22) (layer "B.Cu") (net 23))
 (via (at 133.425 118.4) (size 0.6) (drill 0.3) (layers "F.Cu" "B.Cu") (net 7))
 (segment (start 133.475 119.85) (end 133.475 118.45) (width 0.22) (layer "B.Cu") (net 7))
 (segment (start 133.475 118.45) (end 133.425 118.4) (width 0.22) (layer "B.Cu") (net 7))
 (segment (start 126.325 122.95) (end 126.35 122.925) (width 0.6) (layer "F.Cu") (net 3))
 (segment (start 127.15 119.75) (end 131.25 119.75) (width 0.6) (layer "F.Cu") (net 3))
 (segment (start 135.925 119.265) (end 135.44 119.75) (width 0.6) (layer "F.Cu") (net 3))
 (segment (start 138.54 122.2) (end 139.91 123.57) (width 0.6) (layer "F.Cu") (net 3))
 (segment (start 130.52 119.75) (end 130.525 119.15) (width 0.6) (layer "F.Cu") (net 3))
 (segment (start 135.925 118) (end 135.925 119.265) (width 0.6) (layer "F.Cu") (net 3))
 (segment (start 136.74 119.75) (end 134.797113 119.75) (width 0.4) (layer "F.Cu") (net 3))
 (segment (start 126.35 122.925) (end 126.35 120.55) (width 0.6) (layer "F.Cu") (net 3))
 (segment (start 127.075 122.2) (end 138.54 122.2) (width 0.6) (layer "F.Cu") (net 3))
 (segment (start 130.5 122.2) (end 130.5 123.8) (width 0.6) (layer "F.Cu") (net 3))
 (segment (start 139.36 119.29) (end 137.2 119.29) (width 0.4) (layer "F.Cu") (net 3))
 (segment (start 130.525 119.15) (end 130.525 118) (width 0.6) (layer "F.Cu") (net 3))
 (segment (start 126.325 122.95) (end 127.075 122.2) (width 0.6) (layer "F.Cu") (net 3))
 (segment (start 126.35 120.55) (end 127.15 119.75) (width 0.6) (layer "F.Cu") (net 3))
 (segment (start 126.225 123.025) (end 126.325 122.95) (width 0.6) (layer "F.Cu") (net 3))
 (segment (start 139.91 123.57) (end 139.91 124.7) (width 0.6) (layer "F.Cu") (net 3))
 (segment (start 135.9 122.21) (end 135.9 123.8) (width 0.6) (layer "F.Cu") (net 3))
 (segment (start 134.797113 119.75) (end 130.52 119.75) (width 0.6) (layer "F.Cu") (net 3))
 (segment (start 137.2 119.29) (end 136.74 119.75) (width 0.4) (layer "F.Cu") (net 3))
 (segment (start 135.44 119.75) (end 134.797113 119.75) (width 0.6) (layer "F.Cu") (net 3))
 (via (at 127.05 123.9) (size 0.6) (drill 0.3) (layers "F.Cu" "B.Cu") (free) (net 3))
 (via (at 126.225 123.025) (size 0.6) (drill 0.3) (layers "F.Cu" "B.Cu") (free) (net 3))
 (via (at 126.225 123.9) (size 0.6) (drill 0.3) (layers "F.Cu" "B.Cu") (free) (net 3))
 (via (at 127.05 123.05) (size 0.6) (drill 0.3) (layers "F.Cu" "B.Cu") (free) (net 3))
 (segment (start 131.62 118.92) (end 131.62 117.42) (width 0.22) (layer "F.Cu") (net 18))
 (segment (start 131.62 117.42) (end 131.5 117.3) (width 0.22) (layer "F.Cu") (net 18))
 (segment (start 131.65 118.95) (end 131.62 118.92) (width 0.22) (layer "F.Cu") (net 18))
 (via (at 131.65 118.95) (size 0.6) (drill 0.3) (layers "F.Cu" "B.Cu") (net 18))
 (via (at 131.5 117.3) (size 0.6) (drill 0.3) (layers "F.Cu" "B.Cu") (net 18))
 (segment (start 131.5 117.3) (end 131.875 116.675) (width 0.22) (layer "B.Cu") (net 18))
 (segment (start 131.65 118.95) (end 131.775 119.075) (width 0.22) (layer "B.Cu") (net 18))
 (segment (start 131.775 119.075) (end 131.775 119.85) (width 0.22) (layer "B.Cu") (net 18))
 (segment (start 127.75 116.8) (end 127.15 117.4) (width 0.22) (layer "B.Cu") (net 11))
 (segment (start 129.78 120.81) (end 129.41 120.44) (width 0.22) (layer "B.Cu") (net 11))
 (segment (start 130.89057 120.55) (end 130.63057 120.81) (width 0.22) (layer "B.Cu") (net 11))
 (segment (start 131.775 120.55) (end 130.89057 120.55) (width 0.22) (layer "B.Cu") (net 11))
 (segment (start 128.975 118.47) (end 128.615489 118.534511) (width 0.22) (layer "B.Cu") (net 11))
 (segment (start 129.41 118.905) (end 128.975 118.47) (width 0.22) (layer "B.Cu") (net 11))
 (segment (start 130.63057 120.81) (end 129.78 120.81) (width 0.22) (layer "B.Cu") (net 11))
 (segment (start 129.075 116.8) (end 127.75 116.8) (width 0.22) (layer "B.Cu") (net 11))
 (segment (start 129.41 120.44) (end 129.41 118.905) (width 0.22) (layer "B.Cu") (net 11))
 (segment (start 128.615489 118.534511) (end 127.490489 118.534511) (width 0.22) (layer "B.Cu") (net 11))
 (segment (start 127.490489 118.534511) (end 127.1 118.925) (width 0.22) (layer "B.Cu") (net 11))
 (segment (start 127.15 117.4) (end 127.15 118.875) (width 0.22) (layer "B.Cu") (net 11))
 (segment (start 136.39 121.05) (end 138.115 119.325) (width 0.22) (layer "B.Cu") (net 12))
 (segment (start 138.115 118.755) (end 138.115 119.325) (width 0.22) (layer "B.Cu") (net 12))
 (segment (start 136.91 117.55) (end 138.115 118.755) (width 0.22) (layer "B.Cu") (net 12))
 (segment (start 134.675 121.05) (end 136.39 121.05) (width 0.22) (layer "B.Cu") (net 12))
 (segment (start 138.115 119.325) (end 139.3 119.325) (width 0.22) (layer "B.Cu") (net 12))
 (segment (start 136.43 117.55) (end 136.91 117.55) (width 0.22) (layer "B.Cu") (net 12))
 (segment (start 134.245 116.805) (end 134.89 116.805) (width 0.22) (layer "B.Cu") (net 13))
 (segment (start 134.89 116.805) (end 136.88057 116.805) (width 0.22) (layer "B.Cu") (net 13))
 (segment (start 134.034511 118.147531) (end 134.034511 117.015489) (width 0.22) (layer "B.Cu") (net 13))
 (segment (start 138.05057 117.975) (end 139.3 117.975) (width 0.22) (layer "B.Cu") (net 13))
 (segment (start 130.245 120) (end 130.245 118.75) (width 0.22) (layer "B.Cu") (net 13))
 (segment (start 134.034511 118.147531) (end 133.677469 117.790489) (width 0.22) (layer "B.Cu") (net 13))
 (segment (start 136.88057 116.805) (end 138.05057 117.975) (width 0.22) (layer "B.Cu") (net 13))
 (segment (start 134.034511 117.015489) (end 134.245 116.805) (width 0.22) (layer "B.Cu") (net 13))
 (segment (start 132.984511 117.790489) (end 132.445969 118.329031) (width 0.22) (layer "B.Cu") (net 13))
 (segment (start 133.975 119.36158) (end 134.034511 119.302069) (width 0.22) (layer "B.Cu") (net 13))
 (segment (start 134.034511 119.302069) (end 134.034511 118.147531) (width 0.22) (layer "B.Cu") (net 13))
 (segment (start 133.975 119.85) (end 133.975 119.36158) (width 0.22) (layer "B.Cu") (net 13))
 (segment (start 133.677469 117.790489) (end 132.984511 117.790489) (width 0.22) (layer "B.Cu") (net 13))
 (segment (start 132.445969 118.329031) (end 130.845969 118.329031) (width 0.22) (layer "B.Cu") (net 13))
 (segment (start 134.675 119.265) (end 134.89 119.05) (width 0.22) (layer "B.Cu") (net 20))
 (segment (start 134.675 119.85) (end 134.675 119.265) (width 0.22) (layer "B.Cu") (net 20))
 (segment (start 134.89 119.05) (end 134.89 118.455) (width 0.22) (layer "B.Cu") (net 20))
 (segment (start 123.5025 124.56) (end 123.4875 124.575) (width 0.22) (layer "B.Cu") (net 15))
 (segment (start 131.020489 124.784511) (end 125.204511 124.784511) (width 0.22) (layer "B.Cu") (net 15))
 (segment (start 125.204511 124.784511) (end 124.98 124.56) (width 0.22) (layer "B.Cu") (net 15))
 (segment (start 131.045 124.76) (end 131.020489 124.784511) (width 0.22) (layer "B.Cu") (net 15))
 (segment (start 124.98 124.56) (end 123.5025 124.56) (width 0.22) (layer "B.Cu") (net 15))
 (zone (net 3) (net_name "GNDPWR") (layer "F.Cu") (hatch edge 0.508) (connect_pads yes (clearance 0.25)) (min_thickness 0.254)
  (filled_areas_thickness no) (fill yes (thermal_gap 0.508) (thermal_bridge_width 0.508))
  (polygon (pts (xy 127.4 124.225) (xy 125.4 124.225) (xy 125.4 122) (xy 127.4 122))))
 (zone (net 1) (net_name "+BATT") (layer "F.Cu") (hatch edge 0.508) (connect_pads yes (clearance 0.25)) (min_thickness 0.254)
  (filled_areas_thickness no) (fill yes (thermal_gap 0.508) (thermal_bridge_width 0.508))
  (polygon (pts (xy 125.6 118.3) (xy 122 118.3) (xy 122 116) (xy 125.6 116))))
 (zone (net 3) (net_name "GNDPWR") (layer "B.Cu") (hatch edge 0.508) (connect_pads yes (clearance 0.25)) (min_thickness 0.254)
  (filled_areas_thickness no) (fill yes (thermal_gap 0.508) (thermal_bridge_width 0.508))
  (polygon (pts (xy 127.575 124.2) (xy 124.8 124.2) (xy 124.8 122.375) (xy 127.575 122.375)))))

